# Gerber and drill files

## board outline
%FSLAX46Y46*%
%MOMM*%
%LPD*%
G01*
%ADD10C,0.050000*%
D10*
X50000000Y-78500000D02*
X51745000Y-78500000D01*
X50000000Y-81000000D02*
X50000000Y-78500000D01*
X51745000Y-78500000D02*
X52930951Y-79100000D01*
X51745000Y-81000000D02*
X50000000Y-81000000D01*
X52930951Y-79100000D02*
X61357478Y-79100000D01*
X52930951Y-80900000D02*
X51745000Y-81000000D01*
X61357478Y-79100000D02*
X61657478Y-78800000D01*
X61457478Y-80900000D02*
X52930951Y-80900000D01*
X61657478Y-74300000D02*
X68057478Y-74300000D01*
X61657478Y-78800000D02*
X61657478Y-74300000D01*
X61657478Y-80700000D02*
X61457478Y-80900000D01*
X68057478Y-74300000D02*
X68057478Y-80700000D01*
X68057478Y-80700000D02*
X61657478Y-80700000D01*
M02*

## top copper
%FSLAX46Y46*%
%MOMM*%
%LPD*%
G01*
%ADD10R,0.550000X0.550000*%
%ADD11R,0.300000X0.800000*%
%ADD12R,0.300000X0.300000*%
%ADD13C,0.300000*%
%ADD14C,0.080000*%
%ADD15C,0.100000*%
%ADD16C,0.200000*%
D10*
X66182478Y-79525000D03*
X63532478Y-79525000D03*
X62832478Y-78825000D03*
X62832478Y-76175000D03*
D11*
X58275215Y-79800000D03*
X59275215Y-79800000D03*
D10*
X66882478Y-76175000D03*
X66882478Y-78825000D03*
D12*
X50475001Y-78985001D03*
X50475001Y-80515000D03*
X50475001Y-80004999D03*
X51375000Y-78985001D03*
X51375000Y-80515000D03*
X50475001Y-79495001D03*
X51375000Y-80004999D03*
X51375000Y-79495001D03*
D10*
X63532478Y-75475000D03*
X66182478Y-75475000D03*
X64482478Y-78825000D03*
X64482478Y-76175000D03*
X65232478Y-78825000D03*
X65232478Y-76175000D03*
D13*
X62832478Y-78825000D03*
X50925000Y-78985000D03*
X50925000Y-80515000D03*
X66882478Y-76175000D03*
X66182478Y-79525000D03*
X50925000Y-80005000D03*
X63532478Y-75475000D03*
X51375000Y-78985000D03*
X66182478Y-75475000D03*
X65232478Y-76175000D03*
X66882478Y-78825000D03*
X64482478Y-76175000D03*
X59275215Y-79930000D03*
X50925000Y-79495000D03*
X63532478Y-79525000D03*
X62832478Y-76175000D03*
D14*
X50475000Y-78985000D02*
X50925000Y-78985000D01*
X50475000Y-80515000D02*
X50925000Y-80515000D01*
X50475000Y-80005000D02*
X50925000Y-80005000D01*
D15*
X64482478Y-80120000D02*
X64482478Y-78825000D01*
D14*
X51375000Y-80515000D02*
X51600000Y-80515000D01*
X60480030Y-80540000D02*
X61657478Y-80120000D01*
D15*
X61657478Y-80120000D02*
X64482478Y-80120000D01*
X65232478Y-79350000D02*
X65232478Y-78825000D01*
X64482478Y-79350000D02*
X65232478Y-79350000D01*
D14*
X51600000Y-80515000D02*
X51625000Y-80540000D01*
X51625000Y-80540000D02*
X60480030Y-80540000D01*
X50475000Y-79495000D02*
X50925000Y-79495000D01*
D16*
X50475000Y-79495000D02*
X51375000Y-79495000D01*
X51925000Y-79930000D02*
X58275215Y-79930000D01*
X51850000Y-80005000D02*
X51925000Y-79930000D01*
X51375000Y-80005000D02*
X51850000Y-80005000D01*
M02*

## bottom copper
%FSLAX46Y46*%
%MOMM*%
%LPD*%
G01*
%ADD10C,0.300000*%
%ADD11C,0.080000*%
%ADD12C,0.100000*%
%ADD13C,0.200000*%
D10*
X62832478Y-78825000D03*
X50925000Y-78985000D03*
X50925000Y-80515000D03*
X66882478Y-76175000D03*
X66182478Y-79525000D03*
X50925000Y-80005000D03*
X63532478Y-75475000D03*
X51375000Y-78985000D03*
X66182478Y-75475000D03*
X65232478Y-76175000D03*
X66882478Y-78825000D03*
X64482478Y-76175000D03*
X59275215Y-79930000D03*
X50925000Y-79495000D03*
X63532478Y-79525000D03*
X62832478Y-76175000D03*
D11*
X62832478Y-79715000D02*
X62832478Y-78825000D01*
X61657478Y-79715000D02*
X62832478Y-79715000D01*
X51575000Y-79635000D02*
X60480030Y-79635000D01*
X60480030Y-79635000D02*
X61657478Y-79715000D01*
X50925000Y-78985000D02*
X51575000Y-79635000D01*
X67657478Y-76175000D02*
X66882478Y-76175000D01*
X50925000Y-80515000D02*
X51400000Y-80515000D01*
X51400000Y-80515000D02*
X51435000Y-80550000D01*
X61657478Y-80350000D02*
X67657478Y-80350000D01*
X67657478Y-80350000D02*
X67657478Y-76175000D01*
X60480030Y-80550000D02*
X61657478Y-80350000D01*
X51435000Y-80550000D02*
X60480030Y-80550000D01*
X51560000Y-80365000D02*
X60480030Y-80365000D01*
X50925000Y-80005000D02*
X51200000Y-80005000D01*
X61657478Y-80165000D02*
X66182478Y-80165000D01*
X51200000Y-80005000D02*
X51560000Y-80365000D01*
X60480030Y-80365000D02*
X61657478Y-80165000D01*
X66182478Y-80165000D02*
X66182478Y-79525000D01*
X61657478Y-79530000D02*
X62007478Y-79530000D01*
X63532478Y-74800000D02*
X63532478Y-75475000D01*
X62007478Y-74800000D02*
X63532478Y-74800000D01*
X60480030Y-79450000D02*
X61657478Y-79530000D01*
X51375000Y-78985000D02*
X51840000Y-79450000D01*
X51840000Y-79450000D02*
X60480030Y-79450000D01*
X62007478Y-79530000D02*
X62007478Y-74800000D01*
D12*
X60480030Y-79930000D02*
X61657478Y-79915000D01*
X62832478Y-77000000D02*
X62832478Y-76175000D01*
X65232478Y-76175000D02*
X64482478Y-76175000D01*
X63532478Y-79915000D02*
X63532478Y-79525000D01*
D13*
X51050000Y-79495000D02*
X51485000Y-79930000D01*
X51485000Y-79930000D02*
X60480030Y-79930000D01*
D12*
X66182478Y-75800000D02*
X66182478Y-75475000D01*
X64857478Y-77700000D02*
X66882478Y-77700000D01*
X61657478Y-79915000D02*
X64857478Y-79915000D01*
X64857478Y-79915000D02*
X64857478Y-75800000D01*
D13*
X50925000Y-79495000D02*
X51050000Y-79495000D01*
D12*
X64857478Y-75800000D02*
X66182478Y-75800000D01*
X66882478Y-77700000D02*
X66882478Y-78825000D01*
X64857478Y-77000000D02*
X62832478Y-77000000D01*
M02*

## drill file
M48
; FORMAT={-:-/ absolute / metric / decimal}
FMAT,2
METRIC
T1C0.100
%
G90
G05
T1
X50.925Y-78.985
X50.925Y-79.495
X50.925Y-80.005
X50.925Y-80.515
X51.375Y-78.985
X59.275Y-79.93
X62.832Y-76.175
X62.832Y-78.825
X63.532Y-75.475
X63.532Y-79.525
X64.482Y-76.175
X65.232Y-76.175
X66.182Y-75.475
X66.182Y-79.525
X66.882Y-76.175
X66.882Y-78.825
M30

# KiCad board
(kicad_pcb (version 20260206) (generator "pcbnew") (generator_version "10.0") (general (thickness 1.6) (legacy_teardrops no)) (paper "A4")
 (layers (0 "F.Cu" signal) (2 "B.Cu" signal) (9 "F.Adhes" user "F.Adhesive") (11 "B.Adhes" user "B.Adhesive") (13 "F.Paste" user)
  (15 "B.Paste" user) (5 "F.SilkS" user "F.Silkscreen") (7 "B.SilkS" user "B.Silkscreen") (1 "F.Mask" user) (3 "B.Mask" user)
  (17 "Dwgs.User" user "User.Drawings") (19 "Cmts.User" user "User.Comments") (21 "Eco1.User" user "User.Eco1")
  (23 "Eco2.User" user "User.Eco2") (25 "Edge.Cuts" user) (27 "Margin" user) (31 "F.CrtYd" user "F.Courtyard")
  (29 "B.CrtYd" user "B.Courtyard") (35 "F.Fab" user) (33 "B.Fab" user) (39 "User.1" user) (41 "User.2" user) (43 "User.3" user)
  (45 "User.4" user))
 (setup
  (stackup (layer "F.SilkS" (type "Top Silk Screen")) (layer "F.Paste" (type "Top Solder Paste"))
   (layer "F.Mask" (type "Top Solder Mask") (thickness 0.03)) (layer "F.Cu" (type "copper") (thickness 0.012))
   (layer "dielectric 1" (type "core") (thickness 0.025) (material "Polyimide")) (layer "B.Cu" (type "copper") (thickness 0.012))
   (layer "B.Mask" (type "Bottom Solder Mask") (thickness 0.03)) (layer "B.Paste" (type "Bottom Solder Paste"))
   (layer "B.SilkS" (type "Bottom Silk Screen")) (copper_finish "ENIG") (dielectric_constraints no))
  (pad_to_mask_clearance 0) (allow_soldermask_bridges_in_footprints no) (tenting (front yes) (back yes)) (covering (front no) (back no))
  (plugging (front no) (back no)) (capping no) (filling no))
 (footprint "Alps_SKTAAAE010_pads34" (layer "F.Cu") (at 62.457478 77.5 90)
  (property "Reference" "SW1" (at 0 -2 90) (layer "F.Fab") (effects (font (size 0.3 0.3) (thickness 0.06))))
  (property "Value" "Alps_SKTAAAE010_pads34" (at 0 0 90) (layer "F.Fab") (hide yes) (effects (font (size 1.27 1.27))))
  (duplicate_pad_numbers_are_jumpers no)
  (pad "3" smd rect (at -1.325 0.375 90) (size 0.55 0.55) (layers "F.Cu" "F.Mask") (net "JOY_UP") (solder_mask_margin 0.05)
   (thermal_bridge_angle 45))
  (pad "4" smd rect (at 1.325 0.375 90) (size 0.55 0.55) (layers "F.Cu" "F.Mask") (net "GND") (solder_mask_margin 0.05)
   (thermal_bridge_angle 45)))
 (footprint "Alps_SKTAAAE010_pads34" (layer "F.Cu") (at 64.857478 79.9 180)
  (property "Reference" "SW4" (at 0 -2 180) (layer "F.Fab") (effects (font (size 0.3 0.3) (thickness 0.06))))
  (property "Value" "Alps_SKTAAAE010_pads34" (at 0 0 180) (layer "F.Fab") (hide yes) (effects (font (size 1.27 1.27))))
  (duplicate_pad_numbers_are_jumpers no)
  (pad "3" smd rect (at -1.325 0.375 180) (size 0.55 0.55) (layers "F.Cu" "F.Mask") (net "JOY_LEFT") (solder_mask_margin 0.05)
   (thermal_bridge_angle 45))
  (pad "4" smd rect (at 1.325 0.375 180) (size 0.55 0.55) (layers "F.Cu" "F.Mask") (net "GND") (solder_mask_margin 0.05)
   (thermal_bridge_angle 45)))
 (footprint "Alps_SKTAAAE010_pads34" (layer "F.Cu") (at 67.257478 77.5 -90)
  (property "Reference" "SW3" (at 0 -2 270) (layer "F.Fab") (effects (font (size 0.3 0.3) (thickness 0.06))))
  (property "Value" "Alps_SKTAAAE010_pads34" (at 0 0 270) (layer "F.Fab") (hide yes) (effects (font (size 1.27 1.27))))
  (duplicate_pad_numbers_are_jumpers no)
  (pad "3" smd rect (at -1.325 0.375 270) (size 0.55 0.55) (layers "F.Cu" "F.Mask") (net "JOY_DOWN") (solder_mask_margin 0.05)
   (thermal_bridge_angle 45))
  (pad "4" smd rect (at 1.325 0.375 270) (size 0.55 0.55) (layers "F.Cu" "F.Mask") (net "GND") (solder_mask_margin 0.05)
   (thermal_bridge_angle 45)))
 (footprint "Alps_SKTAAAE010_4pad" (layer "F.Cu") (at 64.857478 77.5 90)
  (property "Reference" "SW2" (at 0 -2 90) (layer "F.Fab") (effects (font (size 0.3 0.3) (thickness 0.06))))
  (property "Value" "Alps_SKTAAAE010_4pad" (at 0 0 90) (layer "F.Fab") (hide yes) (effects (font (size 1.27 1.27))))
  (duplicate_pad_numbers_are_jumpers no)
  (pad "1" smd rect (at -1.325 -0.375 90) (size 0.55 0.55) (layers "F.Cu" "F.Mask") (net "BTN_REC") (solder_mask_margin 0.05)
   (thermal_bridge_angle 45))
  (pad "2" smd rect (at 1.325 -0.375 90) (size 0.55 0.55) (layers "F.Cu" "F.Mask") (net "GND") (solder_mask_margin 0.05)
   (thermal_bridge_angle 45))
  (pad "3" smd rect (at -1.325 0.375 90) (size 0.55 0.55) (layers "F.Cu" "F.Mask") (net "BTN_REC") (solder_mask_margin 0.05)
   (thermal_bridge_angle 45))
  (pad "4" smd rect (at 1.325 0.375 90) (size 0.55 0.55) (layers "F.Cu" "F.Mask") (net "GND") (solder_mask_margin 0.05)
   (thermal_bridge_angle 45)))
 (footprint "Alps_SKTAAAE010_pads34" (layer "F.Cu") (at 64.857478 75.1)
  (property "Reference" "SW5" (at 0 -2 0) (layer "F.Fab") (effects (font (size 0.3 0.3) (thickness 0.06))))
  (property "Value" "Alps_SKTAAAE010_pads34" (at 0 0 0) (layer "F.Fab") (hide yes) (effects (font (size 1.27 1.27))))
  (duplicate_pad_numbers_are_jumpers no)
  (pad "3" smd rect (at -1.325 0.375) (size 0.55 0.55) (layers "F.Cu" "F.Mask") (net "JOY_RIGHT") (solder_mask_margin 0.05)
   (thermal_bridge_angle 45))
  (pad "4" smd rect (at 1.325 0.375) (size 0.55 0.55) (layers "F.Cu" "F.Mask") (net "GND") (solder_mask_margin 0.05)
   (thermal_bridge_angle 45)))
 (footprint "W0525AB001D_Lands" (layer "F.Cu") (at 58.775215 79.93)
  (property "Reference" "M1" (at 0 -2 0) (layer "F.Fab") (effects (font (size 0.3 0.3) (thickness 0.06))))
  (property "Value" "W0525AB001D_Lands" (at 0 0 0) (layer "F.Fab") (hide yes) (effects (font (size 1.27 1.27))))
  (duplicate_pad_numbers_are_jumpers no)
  (pad "1" smd rect (at -0.5 -0.13) (size 0.3 0.8) (layers "F.Cu" "F.Mask") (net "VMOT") (solder_mask_margin 0.05) (thermal_bridge_angle 45))
  (pad "2" smd rect (at 0.5 -0.13) (size 0.3 0.8) (layers "F.Cu" "F.Mask") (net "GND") (solder_mask_margin 0.05) (thermal_bridge_angle 45)))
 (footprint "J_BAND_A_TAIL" (layer "F.Cu") (at 50.9 79.75)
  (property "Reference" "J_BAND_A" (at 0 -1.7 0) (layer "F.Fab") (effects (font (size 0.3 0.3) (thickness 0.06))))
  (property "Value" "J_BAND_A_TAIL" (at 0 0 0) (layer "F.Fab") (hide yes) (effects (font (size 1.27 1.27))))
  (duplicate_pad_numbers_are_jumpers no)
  (pad "1" smd rect (at -0.424999 -0.764999) (size 0.3 0.3) (layers "F.Cu" "F.Mask") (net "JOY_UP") (solder_mask_margin 0.05)
   (thermal_bridge_angle 45))
  (pad "2" smd rect (at -0.424999 0.765) (size 0.3 0.3) (layers "F.Cu" "F.Mask") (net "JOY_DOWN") (solder_mask_margin 0.05)
   (thermal_bridge_angle 45))
  (pad "3" smd rect (at -0.424999 0.254999) (size 0.3 0.3) (layers "F.Cu" "F.Mask") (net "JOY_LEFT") (solder_mask_margin 0.05)
   (thermal_bridge_angle 45))
  (pad "4" smd rect (at 0.475 -0.764999) (size 0.3 0.3) (layers "F.Cu" "F.Mask") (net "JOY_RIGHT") (solder_mask_margin 0.05)
   (thermal_bridge_angle 45))
  (pad "5" smd rect (at 0.475 0.765) (size 0.3 0.3) (layers "F.Cu" "F.Mask") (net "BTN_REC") (solder_mask_margin 0.05)
   (thermal_bridge_angle 45))
  (pad "6" smd rect (at -0.424999 -0.254999) (size 0.3 0.3) (layers "F.Cu" "F.Mask") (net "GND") (solder_mask_margin 0.05)
   (thermal_bridge_angle 45))
  (pad "7" smd rect (at 0.475 0.254999) (size 0.3 0.3) (layers "F.Cu" "F.Mask") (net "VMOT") (solder_mask_margin 0.05)
   (thermal_bridge_angle 45))
  (pad "8" smd rect (at 0.475 -0.254999) (size 0.3 0.3) (layers "F.Cu" "F.Mask") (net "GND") (solder_mask_margin 0.05)
   (thermal_bridge_angle 45)))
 (gr_line (start 50 78.5) (end 51.745 78.5) (stroke (width 0.05) (type default)) (layer "Edge.Cuts"))
 (gr_line (start 50 81) (end 50 78.5) (stroke (width 0.05) (type default)) (layer "Edge.Cuts"))
 (gr_line (start 51.745 78.5) (end 52.930951 79.1) (stroke (width 0.05) (type default)) (layer "Edge.Cuts"))
 (gr_line (start 51.745 81) (end 50 81) (stroke (width 0.05) (type default)) (layer "Edge.Cuts"))
 (gr_line (start 52.930951 79.1) (end 61.357478 79.1) (stroke (width 0.05) (type default)) (layer "Edge.Cuts"))
 (gr_line (start 52.930951 80.9) (end 51.745 81) (stroke (width 0.05) (type default)) (layer "Edge.Cuts"))
 (gr_line (start 61.357478 79.1) (end 61.657478 78.8) (stroke (width 0.05) (type default)) (layer "Edge.Cuts"))
 (gr_line (start 61.457478 80.9) (end 52.930951 80.9) (stroke (width 0.05) (type default)) (layer "Edge.Cuts"))
 (gr_line (start 61.657478 74.3) (end 68.057478 74.3) (stroke (width 0.05) (type default)) (layer "Edge.Cuts"))
 (gr_line (start 61.657478 78.8) (end 61.657478 74.3) (stroke (width 0.05) (type default)) (layer "Edge.Cuts"))
 (gr_line (start 61.657478 80.7) (end 61.457478 80.9) (stroke (width 0.05) (type default)) (layer "Edge.Cuts"))
 (gr_line (start 68.057478 74.3) (end 68.057478 80.7) (stroke (width 0.05) (type default)) (layer "Edge.Cuts"))
 (gr_line (start 68.057478 80.7) (end 61.657478 80.7) (stroke (width 0.05) (type default)) (layer "Edge.Cuts"))
 (segment (start 50.475 78.985) (end 50.925 78.985) (width 0.08) (layer "F.Cu") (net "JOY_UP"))
 (via (at 50.925 78.985) (size 0.3) (drill 0.1) (layers "F.Cu" "B.Cu") (tenting (front yes) (back yes)) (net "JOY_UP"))
 (via (at 62.832478 78.825) (size 0.3) (drill 0.1) (layers "F.Cu" "B.Cu") (tenting (front yes) (back yes)) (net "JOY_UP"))
 (segment (start 50.925 78.985) (end 51.575 79.635) (width 0.08) (layer "B.Cu") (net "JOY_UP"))
 (segment (start 61.657478 79.715) (end 62.832478 79.715) (width 0.08) (layer "B.Cu") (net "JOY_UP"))
 (segment (start 51.575 79.635) (end 60.48003 79.635) (width 0.08) (layer "B.Cu") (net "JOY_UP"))
 (segment (start 62.832478 79.715) (end 62.832478 78.825) (width 0.08) (layer "B.Cu") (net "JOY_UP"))
 (segment (start 60.48003 79.635) (end 61.657478 79.715) (width 0.08) (layer "B.Cu") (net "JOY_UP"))
 (segment (start 50.475 80.515) (end 50.925 80.515) (width 0.08) (layer "F.Cu") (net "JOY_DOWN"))
 (via (at 50.925 80.515) (size 0.3) (drill 0.1) (layers "F.Cu" "B.Cu") (tenting (front yes) (back yes)) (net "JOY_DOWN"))
 (via (at 66.882478 76.175) (size 0.3) (drill 0.1) (layers "F.Cu" "B.Cu") (tenting (front yes) (back yes)) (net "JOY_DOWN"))
 (segment (start 51.435 80.55) (end 60.48003 80.55) (width 0.08) (layer "B.Cu") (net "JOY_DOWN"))
 (segment (start 50.925 80.515) (end 51.4 80.515) (width 0.08) (layer "B.Cu") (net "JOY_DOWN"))
 (segment (start 51.4 80.515) (end 51.435 80.55) (width 0.08) (layer "B.Cu") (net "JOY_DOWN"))
 (segment (start 60.48003 80.55) (end 61.657478 80.35) (width 0.08) (layer "B.Cu") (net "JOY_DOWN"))
 (segment (start 67.657478 76.175) (end 66.882478 76.175) (width 0.08) (layer "B.Cu") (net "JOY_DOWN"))
 (segment (start 61.657478 80.35) (end 67.657478 80.35) (width 0.08) (layer "B.Cu") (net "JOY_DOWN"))
 (segment (start 67.657478 80.35) (end 67.657478 76.175) (width 0.08) (layer "B.Cu") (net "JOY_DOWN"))
 (segment (start 50.475 80.005) (end 50.925 80.005) (width 0.08) (layer "F.Cu") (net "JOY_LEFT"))
 (via (at 66.182478 79.525) (size 0.3) (drill 0.1) (layers "F.Cu" "B.Cu") (tenting (front yes) (back yes)) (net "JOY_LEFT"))
 (via (at 50.925 80.005) (size 0.3) (drill 0.1) (layers "F.Cu" "B.Cu") (tenting (front yes) (back yes)) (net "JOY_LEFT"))
 (segment (start 50.925 80.005) (end 51.2 80.005) (width 0.08) (layer "B.Cu") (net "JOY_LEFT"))
 (segment (start 60.48003 80.365) (end 61.657478 80.165) (width 0.08) (layer "B.Cu") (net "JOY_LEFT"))
 (segment (start 51.2 80.005) (end 51.56 80.365) (width 0.08) (layer "B.Cu") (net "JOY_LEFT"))
 (segment (start 61.657478 80.165) (end 66.182478 80.165) (width 0.08) (layer "B.Cu") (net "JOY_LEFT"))
 (segment (start 66.182478 80.165) (end 66.182478 79.525) (width 0.08) (layer "B.Cu") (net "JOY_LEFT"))
 (segment (start 51.56 80.365) (end 60.48003 80.365) (width 0.08) (layer "B.Cu") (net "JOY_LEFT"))
 (via (at 63.532478 75.475) (size 0.3) (drill 0.1) (layers "F.Cu" "B.Cu") (tenting (front yes) (back yes)) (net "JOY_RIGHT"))
 (via (at 51.375 78.985) (size 0.3) (drill 0.1) (layers "F.Cu" "B.Cu") (tenting (front yes) (back yes)) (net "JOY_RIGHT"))
 (segment (start 60.48003 79.45) (end 61.657478 79.53) (width 0.08) (layer "B.Cu") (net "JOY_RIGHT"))
 (segment (start 63.532478 74.8) (end 63.532478 75.475) (width 0.08) (layer "B.Cu") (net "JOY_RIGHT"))
 (segment (start 62.007478 74.8) (end 63.532478 74.8) (width 0.08) (layer "B.Cu") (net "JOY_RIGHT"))
 (segment (start 62.007478 79.53) (end 62.007478 74.8) (width 0.08) (layer "B.Cu") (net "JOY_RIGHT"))
 (segment (start 51.375 78.985) (end 51.84 79.45) (width 0.08) (layer "B.Cu") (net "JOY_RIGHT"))
 (segment (start 51.84 79.45) (end 60.48003 79.45) (width 0.08) (layer "B.Cu") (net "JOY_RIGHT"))
 (segment (start 61.657478 79.53) (end 62.007478 79.53) (width 0.08) (layer "B.Cu") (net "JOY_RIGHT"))
 (segment (start 64.482478 79.35) (end 65.232478 79.35) (width 0.1) (layer "F.Cu") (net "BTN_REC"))
 (segment (start 60.48003 80.54) (end 61.657478 80.12) (width 0.08) (layer "F.Cu") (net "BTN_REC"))
 (segment (start 51.625 80.54) (end 60.48003 80.54) (width 0.08) (layer "F.Cu") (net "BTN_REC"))
 (segment (start 51.6 80.515) (end 51.625 80.54) (width 0.08) (layer "F.Cu") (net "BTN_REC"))
 (segment (start 64.482478 80.12) (end 64.482478 78.825) (width 0.1) (layer "F.Cu") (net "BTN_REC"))
 (segment (start 61.657478 80.12) (end 64.482478 80.12) (width 0.1) (layer "F.Cu") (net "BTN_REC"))
 (segment (start 65.232478 79.35) (end 65.232478 78.825) (width 0.1) (layer "F.Cu") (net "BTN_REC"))
 (segment (start 51.375 80.515) (end 51.6 80.515) (width 0.08) (layer "F.Cu") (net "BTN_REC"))
 (segment (start 50.475 79.495) (end 50.925 79.495) (width 0.08) (layer "F.Cu") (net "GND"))
 (segment (start 50.475 79.495) (end 51.375 79.495) (width 0.2) (layer "F.Cu") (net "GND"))
 (via (at 62.832478 76.175) (size 0.3) (drill 0.1) (layers "F.Cu" "B.Cu") (tenting (front yes) (back yes)) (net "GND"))
 (via (at 59.275215 79.93) (size 0.3) (drill 0.1) (layers "F.Cu" "B.Cu") (tenting (front yes) (back yes)) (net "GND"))
 (via (at 66.882478 78.825) (size 0.3) (drill 0.1) (layers "F.Cu" "B.Cu") (tenting (front yes) (back yes)) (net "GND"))
 (via (at 66.182478 75.475) (size 0.3) (drill 0.1) (layers "F.Cu" "B.Cu") (tenting (front yes) (back yes)) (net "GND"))
 (via (at 50.925 79.495) (size 0.3) (drill 0.1) (layers "F.Cu" "B.Cu") (tenting (front yes) (back yes)) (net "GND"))
 (via (at 65.232478 76.175) (size 0.3) (drill 0.1) (layers "F.Cu" "B.Cu") (tenting (front yes) (back yes)) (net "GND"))
 (via (at 64.482478 76.175) (size 0.3) (drill 0.1) (layers "F.Cu" "B.Cu") (tenting (front yes) (back yes)) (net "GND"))
 (via (at 63.532478 79.525) (size 0.3) (drill 0.1) (layers "F.Cu" "B.Cu") (tenting (front yes) (back yes)) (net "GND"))
 (segment (start 64.857478 79.915) (end 64.857478 75.8) (width 0.1) (layer "B.Cu") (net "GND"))
 (segment (start 66.882478 77.7) (end 66.882478 78.825) (width 0.1) (layer "B.Cu") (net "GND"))
 (segment (start 51.485 79.93) (end 60.48003 79.93) (width 0.2) (layer "B.Cu") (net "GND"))
 (segment (start 64.857478 75.8) (end 66.182478 75.8) (width 0.1) (layer "B.Cu") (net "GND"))
 (segment (start 64.857478 77.7) (end 66.882478 77.7) (width 0.1) (layer "B.Cu") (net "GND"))
 (segment (start 66.182478 75.8) (end 66.182478 75.475) (width 0.1) (layer "B.Cu") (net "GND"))
 (segment (start 61.657478 79.915) (end 64.857478 79.915) (width 0.1) (layer "B.Cu") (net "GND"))
 (segment (start 62.832478 77) (end 62.832478 76.175) (width 0.1) (layer "B.Cu") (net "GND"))
 (segment (start 51.05 79.495) (end 51.485 79.93) (width 0.2) (layer "B.Cu") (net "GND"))
 (segment (start 63.532478 79.915) (end 63.532478 79.525) (width 0.1) (layer "B.Cu") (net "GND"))
 (segment (start 64.857478 77) (end 62.832478 77) (width 0.1) (layer "B.Cu") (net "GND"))
 (segment (start 50.925 79.495) (end 51.05 79.495) (width 0.2) (layer "B.Cu") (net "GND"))
 (segment (start 65.232478 76.175) (end 64.482478 76.175) (width 0.1) (layer "B.Cu") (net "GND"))
 (segment (start 60.48003 79.93) (end 61.657478 79.915) (width 0.1) (layer "B.Cu") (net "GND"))
 (segment (start 51.375 80.005) (end 51.85 80.005) (width 0.2) (layer "F.Cu") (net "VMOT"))
 (segment (start 51.85 80.005) (end 51.925 79.93) (width 0.2) (layer "F.Cu") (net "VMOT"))
 (segment (start 51.925 79.93) (end 58.275215 79.93) (width 0.2) (layer "F.Cu") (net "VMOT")))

